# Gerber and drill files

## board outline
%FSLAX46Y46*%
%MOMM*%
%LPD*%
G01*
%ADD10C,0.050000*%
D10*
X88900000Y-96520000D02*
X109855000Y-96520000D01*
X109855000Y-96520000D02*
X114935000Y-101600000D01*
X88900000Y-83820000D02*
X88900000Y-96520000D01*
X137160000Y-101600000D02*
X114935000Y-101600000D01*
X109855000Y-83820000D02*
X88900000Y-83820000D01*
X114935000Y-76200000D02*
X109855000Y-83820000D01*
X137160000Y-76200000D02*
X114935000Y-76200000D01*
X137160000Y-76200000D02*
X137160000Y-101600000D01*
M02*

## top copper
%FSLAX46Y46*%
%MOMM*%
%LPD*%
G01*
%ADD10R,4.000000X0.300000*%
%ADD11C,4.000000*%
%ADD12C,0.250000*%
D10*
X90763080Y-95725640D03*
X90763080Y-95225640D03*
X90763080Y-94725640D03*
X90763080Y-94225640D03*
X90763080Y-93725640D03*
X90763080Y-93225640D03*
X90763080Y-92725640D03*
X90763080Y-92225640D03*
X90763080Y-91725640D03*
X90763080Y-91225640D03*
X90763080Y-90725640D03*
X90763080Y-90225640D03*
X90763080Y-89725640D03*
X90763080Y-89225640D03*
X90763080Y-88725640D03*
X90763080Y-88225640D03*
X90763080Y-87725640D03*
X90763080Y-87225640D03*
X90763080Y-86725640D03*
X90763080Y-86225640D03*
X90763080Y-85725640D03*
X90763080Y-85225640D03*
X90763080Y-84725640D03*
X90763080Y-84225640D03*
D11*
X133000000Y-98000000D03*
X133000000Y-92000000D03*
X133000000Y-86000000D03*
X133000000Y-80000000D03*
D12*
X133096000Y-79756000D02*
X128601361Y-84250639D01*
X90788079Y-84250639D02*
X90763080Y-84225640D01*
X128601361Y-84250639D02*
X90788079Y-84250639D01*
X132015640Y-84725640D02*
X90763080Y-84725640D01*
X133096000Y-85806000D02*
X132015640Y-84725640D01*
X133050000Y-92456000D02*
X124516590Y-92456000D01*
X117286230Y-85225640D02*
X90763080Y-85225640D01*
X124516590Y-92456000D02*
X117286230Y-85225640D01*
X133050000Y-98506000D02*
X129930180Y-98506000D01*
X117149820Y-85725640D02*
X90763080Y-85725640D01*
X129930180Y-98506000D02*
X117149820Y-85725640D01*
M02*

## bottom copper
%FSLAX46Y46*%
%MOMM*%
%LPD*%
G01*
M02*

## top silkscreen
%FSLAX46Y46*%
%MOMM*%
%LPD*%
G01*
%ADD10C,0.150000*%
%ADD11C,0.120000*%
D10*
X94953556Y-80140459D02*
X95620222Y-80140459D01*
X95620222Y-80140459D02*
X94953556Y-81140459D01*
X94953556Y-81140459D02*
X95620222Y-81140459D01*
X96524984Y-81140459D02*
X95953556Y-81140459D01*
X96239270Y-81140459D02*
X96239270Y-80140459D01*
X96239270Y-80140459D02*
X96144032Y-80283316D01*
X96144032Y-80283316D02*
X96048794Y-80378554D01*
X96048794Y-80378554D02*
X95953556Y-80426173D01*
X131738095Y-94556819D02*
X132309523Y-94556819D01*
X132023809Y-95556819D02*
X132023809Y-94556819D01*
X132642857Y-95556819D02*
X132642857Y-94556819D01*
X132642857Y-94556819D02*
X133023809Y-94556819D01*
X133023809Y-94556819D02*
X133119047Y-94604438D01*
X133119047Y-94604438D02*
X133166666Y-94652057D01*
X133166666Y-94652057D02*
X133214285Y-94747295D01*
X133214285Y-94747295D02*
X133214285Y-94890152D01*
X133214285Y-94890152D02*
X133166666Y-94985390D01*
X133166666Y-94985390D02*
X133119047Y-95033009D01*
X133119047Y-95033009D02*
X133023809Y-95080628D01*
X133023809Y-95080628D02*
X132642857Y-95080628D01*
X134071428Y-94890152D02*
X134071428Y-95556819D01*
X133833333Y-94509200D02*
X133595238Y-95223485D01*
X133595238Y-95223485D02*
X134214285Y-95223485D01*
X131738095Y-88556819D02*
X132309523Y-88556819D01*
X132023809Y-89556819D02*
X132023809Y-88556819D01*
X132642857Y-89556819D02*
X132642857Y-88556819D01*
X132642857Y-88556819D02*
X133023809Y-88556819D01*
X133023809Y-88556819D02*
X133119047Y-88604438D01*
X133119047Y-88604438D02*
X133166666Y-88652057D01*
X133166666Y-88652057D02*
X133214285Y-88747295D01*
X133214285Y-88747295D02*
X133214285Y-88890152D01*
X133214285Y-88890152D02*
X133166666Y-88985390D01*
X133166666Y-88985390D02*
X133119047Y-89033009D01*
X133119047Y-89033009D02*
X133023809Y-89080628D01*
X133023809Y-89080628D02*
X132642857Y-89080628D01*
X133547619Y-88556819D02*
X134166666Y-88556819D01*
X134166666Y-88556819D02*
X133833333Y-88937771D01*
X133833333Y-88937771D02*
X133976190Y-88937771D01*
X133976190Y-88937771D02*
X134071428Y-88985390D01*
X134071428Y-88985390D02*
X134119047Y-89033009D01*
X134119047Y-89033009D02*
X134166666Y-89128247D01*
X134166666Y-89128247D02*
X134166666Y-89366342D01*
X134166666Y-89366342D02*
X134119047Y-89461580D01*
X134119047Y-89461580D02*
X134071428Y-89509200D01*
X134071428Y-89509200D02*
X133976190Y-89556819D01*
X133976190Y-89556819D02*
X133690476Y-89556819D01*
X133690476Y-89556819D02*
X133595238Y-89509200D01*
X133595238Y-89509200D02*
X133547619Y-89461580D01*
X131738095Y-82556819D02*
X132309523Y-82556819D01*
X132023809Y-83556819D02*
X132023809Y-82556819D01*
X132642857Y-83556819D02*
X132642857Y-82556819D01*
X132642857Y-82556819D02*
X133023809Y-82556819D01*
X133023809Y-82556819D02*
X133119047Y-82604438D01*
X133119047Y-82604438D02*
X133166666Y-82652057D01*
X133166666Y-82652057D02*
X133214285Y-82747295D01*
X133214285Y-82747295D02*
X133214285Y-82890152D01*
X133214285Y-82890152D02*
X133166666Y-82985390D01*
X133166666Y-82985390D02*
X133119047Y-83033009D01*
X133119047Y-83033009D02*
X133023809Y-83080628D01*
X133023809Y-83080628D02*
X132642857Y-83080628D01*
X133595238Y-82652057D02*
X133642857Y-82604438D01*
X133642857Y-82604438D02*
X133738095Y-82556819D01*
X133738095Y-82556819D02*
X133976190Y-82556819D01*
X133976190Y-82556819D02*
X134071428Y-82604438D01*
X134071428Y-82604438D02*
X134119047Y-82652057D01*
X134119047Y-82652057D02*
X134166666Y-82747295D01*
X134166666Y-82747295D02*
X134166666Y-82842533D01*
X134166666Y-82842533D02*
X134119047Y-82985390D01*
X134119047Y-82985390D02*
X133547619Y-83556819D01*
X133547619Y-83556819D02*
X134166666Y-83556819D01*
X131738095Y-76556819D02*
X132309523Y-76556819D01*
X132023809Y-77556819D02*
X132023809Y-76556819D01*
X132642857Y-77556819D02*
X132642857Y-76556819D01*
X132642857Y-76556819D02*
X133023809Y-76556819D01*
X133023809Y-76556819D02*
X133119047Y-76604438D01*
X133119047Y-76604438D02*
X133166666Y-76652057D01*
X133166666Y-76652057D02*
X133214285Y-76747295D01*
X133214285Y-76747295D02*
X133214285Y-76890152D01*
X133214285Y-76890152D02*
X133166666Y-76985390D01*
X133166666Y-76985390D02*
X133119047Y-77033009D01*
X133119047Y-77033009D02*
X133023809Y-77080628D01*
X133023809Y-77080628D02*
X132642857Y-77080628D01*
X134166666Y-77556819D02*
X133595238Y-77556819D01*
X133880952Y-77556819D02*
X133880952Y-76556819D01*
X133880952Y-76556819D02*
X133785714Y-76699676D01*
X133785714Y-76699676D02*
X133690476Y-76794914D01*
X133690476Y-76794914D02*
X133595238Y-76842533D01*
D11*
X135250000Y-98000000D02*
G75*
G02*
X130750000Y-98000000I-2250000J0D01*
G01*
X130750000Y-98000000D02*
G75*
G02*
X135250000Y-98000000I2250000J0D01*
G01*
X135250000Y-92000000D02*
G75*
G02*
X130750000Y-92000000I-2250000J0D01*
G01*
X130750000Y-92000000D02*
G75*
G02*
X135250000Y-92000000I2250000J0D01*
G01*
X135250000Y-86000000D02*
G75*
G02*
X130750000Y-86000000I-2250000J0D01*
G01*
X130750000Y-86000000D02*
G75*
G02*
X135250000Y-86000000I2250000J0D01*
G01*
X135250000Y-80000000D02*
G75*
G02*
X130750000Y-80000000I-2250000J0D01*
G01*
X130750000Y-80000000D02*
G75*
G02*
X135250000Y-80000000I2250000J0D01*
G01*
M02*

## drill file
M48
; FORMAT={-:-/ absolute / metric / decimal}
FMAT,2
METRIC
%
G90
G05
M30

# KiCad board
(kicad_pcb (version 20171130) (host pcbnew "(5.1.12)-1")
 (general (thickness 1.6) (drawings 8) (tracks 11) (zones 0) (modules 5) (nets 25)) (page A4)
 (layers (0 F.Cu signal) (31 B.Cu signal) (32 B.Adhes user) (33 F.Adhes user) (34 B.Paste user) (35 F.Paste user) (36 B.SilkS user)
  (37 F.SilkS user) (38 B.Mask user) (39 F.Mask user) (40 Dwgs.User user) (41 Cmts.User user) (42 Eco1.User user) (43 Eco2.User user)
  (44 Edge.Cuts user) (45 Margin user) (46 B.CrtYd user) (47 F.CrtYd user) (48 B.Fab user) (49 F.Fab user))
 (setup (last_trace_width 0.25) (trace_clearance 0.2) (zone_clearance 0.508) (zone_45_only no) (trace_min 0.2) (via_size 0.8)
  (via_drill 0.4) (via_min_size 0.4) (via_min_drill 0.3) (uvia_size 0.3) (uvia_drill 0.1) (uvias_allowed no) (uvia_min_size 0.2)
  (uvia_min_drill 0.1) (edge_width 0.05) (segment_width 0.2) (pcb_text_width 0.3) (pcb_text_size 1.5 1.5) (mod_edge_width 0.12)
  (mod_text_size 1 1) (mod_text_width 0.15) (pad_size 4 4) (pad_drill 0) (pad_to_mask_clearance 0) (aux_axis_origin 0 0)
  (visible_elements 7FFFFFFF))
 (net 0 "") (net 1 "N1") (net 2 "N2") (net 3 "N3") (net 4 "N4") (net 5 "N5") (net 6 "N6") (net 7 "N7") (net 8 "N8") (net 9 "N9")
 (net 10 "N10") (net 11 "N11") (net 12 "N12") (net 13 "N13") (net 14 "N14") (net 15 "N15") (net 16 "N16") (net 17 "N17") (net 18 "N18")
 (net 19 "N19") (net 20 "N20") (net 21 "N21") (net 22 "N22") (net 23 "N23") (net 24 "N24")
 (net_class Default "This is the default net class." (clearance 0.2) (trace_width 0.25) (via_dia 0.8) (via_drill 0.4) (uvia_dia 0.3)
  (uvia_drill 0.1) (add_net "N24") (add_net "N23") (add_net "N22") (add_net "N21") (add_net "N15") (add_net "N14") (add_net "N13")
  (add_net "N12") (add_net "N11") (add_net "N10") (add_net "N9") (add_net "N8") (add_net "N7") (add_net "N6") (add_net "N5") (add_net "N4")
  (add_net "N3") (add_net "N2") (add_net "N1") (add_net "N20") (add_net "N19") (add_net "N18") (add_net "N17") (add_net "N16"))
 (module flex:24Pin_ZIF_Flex (layer F.Cu) (at 95.76308 83.22564) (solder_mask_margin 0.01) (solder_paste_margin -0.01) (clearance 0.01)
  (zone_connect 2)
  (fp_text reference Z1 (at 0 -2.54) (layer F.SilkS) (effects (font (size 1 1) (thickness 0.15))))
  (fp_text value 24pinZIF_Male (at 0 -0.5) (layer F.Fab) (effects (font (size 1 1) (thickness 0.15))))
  (pad 24 connect rect (at -5 12.5) (size 4 0.3) (layers F.Cu F.Mask) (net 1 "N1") (zone_connect 2))
  (pad 23 connect rect (at -5 12) (size 4 0.3) (layers F.Cu F.Mask) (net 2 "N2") (zone_connect 2))
  (pad 22 connect rect (at -5 11.5) (size 4 0.3) (layers F.Cu F.Mask) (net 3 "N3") (zone_connect 2))
  (pad 21 connect rect (at -5 11) (size 4 0.3) (layers F.Cu F.Mask) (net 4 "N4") (zone_connect 2))
  (pad 20 connect rect (at -5 10.5) (size 4 0.3) (layers F.Cu F.Mask) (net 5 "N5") (zone_connect 2))
  (pad 19 connect rect (at -5 10) (size 4 0.3) (layers F.Cu F.Mask) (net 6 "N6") (zone_connect 2))
  (pad 18 connect rect (at -5 9.5) (size 4 0.3) (layers F.Cu F.Mask) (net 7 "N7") (zone_connect 2))
  (pad 17 connect rect (at -5 9) (size 4 0.3) (layers F.Cu F.Mask) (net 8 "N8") (zone_connect 2))
  (pad 16 connect rect (at -5 8.5) (size 4 0.3) (layers F.Cu F.Mask) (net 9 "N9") (zone_connect 2))
  (pad 15 connect rect (at -5 8) (size 4 0.3) (layers F.Cu F.Mask) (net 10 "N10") (zone_connect 2))
  (pad 14 connect rect (at -5 7.5) (size 4 0.3) (layers F.Cu F.Mask) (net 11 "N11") (zone_connect 2))
  (pad 13 connect rect (at -5 7) (size 4 0.3) (layers F.Cu F.Mask) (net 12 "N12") (zone_connect 2))
  (pad 12 connect rect (at -5 6.5) (size 4 0.3) (layers F.Cu F.Mask) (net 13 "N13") (zone_connect 2))
  (pad 11 connect rect (at -5 6) (size 4 0.3) (layers F.Cu F.Mask) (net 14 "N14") (zone_connect 2))
  (pad 10 connect rect (at -5 5.5) (size 4 0.3) (layers F.Cu F.Mask) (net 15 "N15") (zone_connect 2))
  (pad 9 connect rect (at -5 5) (size 4 0.3) (layers F.Cu F.Mask) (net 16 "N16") (zone_connect 2))
  (pad 8 connect rect (at -5 4.5) (size 4 0.3) (layers F.Cu F.Mask) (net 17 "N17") (zone_connect 2))
  (pad 7 connect rect (at -5 4) (size 4 0.3) (layers F.Cu F.Mask) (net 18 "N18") (zone_connect 2))
  (pad 6 connect rect (at -5 3.5) (size 4 0.3) (layers F.Cu F.Mask) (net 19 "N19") (zone_connect 2))
  (pad 5 connect rect (at -5 3) (size 4 0.3) (layers F.Cu F.Mask) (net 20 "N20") (zone_connect 2))
  (pad 4 connect rect (at -5 2.5) (size 4 0.3) (layers F.Cu F.Mask) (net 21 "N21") (zone_connect 2))
  (pad 3 connect rect (at -5 2) (size 4 0.3) (layers F.Cu F.Mask) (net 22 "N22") (zone_connect 2))
  (pad 2 connect rect (at -5 1.5) (size 4 0.3) (layers F.Cu F.Mask) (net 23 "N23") (zone_connect 2))
  (pad 1 connect rect (at -5 1) (size 4 0.3) (layers F.Cu F.Mask) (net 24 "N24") (zone_connect 2)))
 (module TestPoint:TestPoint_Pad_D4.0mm (layer F.Cu) (at 133 98)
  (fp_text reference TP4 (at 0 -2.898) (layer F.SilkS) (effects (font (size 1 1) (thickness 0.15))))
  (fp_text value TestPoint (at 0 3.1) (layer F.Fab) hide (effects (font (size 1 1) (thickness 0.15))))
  (fp_circle (center 0 0) (end 0 2.25) (layer F.SilkS) (width 0.12))
  (pad 1 smd circle (at 0 0) (size 4 4) (layers F.Cu F.Mask) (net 21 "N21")))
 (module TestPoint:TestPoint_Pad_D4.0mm (layer F.Cu) (at 133 92)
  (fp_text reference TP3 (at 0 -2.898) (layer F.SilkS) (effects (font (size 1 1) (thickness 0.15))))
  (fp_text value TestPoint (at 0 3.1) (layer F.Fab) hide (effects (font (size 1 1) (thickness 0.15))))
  (fp_circle (center 0 0) (end 0 2.25) (layer F.SilkS) (width 0.12))
  (pad 1 smd circle (at 0 0) (size 4 4) (layers F.Cu F.Mask) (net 22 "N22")))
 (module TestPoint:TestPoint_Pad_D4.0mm (layer F.Cu) (at 133 86)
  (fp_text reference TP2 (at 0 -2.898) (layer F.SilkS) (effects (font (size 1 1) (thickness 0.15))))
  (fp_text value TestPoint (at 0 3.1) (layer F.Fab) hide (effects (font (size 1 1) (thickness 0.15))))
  (fp_circle (center 0 0) (end 0 2.25) (layer F.SilkS) (width 0.12))
  (pad 1 smd circle (at 0 0) (size 4 4) (layers F.Cu F.Mask) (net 23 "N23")))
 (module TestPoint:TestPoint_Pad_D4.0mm (layer F.Cu) (at 133 80)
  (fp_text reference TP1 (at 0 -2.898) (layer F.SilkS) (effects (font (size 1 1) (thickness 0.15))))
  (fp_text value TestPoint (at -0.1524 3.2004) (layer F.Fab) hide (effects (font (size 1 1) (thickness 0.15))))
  (fp_circle (center 0 0) (end 0 2.25) (layer F.SilkS) (width 0.12))
  (pad 1 smd circle (at 0 0) (size 4 4) (layers F.Cu F.Mask) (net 24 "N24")))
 (gr_line (start 88.9 96.52) (end 109.855 96.52) (layer Edge.Cuts) (width 0.05))
 (gr_line (start 109.855 96.52) (end 114.935 101.6) (layer Edge.Cuts) (width 0.05))
 (gr_line (start 88.9 83.82) (end 88.9 96.52) (layer Edge.Cuts) (width 0.05))
 (gr_line (start 137.16 101.6) (end 114.935 101.6) (layer Edge.Cuts) (width 0.05))
 (gr_line (start 109.855 83.82) (end 88.9 83.82) (layer Edge.Cuts) (width 0.05))
 (gr_line (start 114.935 76.2) (end 109.855 83.82) (layer Edge.Cuts) (width 0.05))
 (gr_line (start 137.16 76.2) (end 114.935 76.2) (layer Edge.Cuts) (width 0.05))
 (gr_line (start 137.16 76.2) (end 137.16 101.6) (layer Edge.Cuts) (width 0.05))
 (segment (start 133.096 79.756) (end 128.601361 84.250639) (width 0.25) (layer F.Cu) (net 24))
 (segment (start 90.788079 84.250639) (end 90.76308 84.22564) (width 0.25) (layer F.Cu) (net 24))
 (segment (start 128.601361 84.250639) (end 90.788079 84.250639) (width 0.25) (layer F.Cu) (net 24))
 (segment (start 132.01564 84.72564) (end 90.76308 84.72564) (width 0.25) (layer F.Cu) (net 23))
 (segment (start 133.096 85.806) (end 132.01564 84.72564) (width 0.25) (layer F.Cu) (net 23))
 (segment (start 133.05 92.456) (end 124.51659 92.456) (width 0.25) (layer F.Cu) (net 22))
 (segment (start 117.28623 85.22564) (end 90.76308 85.22564) (width 0.25) (layer F.Cu) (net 22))
 (segment (start 124.51659 92.456) (end 117.28623 85.22564) (width 0.25) (layer F.Cu) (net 22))
 (segment (start 133.05 98.506) (end 129.93018 98.506) (width 0.25) (layer F.Cu) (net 21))
 (segment (start 117.14982 85.72564) (end 90.76308 85.72564) (width 0.25) (layer F.Cu) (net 21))
 (segment (start 129.93018 98.506) (end 117.14982 85.72564) (width 0.25) (layer F.Cu) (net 21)))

